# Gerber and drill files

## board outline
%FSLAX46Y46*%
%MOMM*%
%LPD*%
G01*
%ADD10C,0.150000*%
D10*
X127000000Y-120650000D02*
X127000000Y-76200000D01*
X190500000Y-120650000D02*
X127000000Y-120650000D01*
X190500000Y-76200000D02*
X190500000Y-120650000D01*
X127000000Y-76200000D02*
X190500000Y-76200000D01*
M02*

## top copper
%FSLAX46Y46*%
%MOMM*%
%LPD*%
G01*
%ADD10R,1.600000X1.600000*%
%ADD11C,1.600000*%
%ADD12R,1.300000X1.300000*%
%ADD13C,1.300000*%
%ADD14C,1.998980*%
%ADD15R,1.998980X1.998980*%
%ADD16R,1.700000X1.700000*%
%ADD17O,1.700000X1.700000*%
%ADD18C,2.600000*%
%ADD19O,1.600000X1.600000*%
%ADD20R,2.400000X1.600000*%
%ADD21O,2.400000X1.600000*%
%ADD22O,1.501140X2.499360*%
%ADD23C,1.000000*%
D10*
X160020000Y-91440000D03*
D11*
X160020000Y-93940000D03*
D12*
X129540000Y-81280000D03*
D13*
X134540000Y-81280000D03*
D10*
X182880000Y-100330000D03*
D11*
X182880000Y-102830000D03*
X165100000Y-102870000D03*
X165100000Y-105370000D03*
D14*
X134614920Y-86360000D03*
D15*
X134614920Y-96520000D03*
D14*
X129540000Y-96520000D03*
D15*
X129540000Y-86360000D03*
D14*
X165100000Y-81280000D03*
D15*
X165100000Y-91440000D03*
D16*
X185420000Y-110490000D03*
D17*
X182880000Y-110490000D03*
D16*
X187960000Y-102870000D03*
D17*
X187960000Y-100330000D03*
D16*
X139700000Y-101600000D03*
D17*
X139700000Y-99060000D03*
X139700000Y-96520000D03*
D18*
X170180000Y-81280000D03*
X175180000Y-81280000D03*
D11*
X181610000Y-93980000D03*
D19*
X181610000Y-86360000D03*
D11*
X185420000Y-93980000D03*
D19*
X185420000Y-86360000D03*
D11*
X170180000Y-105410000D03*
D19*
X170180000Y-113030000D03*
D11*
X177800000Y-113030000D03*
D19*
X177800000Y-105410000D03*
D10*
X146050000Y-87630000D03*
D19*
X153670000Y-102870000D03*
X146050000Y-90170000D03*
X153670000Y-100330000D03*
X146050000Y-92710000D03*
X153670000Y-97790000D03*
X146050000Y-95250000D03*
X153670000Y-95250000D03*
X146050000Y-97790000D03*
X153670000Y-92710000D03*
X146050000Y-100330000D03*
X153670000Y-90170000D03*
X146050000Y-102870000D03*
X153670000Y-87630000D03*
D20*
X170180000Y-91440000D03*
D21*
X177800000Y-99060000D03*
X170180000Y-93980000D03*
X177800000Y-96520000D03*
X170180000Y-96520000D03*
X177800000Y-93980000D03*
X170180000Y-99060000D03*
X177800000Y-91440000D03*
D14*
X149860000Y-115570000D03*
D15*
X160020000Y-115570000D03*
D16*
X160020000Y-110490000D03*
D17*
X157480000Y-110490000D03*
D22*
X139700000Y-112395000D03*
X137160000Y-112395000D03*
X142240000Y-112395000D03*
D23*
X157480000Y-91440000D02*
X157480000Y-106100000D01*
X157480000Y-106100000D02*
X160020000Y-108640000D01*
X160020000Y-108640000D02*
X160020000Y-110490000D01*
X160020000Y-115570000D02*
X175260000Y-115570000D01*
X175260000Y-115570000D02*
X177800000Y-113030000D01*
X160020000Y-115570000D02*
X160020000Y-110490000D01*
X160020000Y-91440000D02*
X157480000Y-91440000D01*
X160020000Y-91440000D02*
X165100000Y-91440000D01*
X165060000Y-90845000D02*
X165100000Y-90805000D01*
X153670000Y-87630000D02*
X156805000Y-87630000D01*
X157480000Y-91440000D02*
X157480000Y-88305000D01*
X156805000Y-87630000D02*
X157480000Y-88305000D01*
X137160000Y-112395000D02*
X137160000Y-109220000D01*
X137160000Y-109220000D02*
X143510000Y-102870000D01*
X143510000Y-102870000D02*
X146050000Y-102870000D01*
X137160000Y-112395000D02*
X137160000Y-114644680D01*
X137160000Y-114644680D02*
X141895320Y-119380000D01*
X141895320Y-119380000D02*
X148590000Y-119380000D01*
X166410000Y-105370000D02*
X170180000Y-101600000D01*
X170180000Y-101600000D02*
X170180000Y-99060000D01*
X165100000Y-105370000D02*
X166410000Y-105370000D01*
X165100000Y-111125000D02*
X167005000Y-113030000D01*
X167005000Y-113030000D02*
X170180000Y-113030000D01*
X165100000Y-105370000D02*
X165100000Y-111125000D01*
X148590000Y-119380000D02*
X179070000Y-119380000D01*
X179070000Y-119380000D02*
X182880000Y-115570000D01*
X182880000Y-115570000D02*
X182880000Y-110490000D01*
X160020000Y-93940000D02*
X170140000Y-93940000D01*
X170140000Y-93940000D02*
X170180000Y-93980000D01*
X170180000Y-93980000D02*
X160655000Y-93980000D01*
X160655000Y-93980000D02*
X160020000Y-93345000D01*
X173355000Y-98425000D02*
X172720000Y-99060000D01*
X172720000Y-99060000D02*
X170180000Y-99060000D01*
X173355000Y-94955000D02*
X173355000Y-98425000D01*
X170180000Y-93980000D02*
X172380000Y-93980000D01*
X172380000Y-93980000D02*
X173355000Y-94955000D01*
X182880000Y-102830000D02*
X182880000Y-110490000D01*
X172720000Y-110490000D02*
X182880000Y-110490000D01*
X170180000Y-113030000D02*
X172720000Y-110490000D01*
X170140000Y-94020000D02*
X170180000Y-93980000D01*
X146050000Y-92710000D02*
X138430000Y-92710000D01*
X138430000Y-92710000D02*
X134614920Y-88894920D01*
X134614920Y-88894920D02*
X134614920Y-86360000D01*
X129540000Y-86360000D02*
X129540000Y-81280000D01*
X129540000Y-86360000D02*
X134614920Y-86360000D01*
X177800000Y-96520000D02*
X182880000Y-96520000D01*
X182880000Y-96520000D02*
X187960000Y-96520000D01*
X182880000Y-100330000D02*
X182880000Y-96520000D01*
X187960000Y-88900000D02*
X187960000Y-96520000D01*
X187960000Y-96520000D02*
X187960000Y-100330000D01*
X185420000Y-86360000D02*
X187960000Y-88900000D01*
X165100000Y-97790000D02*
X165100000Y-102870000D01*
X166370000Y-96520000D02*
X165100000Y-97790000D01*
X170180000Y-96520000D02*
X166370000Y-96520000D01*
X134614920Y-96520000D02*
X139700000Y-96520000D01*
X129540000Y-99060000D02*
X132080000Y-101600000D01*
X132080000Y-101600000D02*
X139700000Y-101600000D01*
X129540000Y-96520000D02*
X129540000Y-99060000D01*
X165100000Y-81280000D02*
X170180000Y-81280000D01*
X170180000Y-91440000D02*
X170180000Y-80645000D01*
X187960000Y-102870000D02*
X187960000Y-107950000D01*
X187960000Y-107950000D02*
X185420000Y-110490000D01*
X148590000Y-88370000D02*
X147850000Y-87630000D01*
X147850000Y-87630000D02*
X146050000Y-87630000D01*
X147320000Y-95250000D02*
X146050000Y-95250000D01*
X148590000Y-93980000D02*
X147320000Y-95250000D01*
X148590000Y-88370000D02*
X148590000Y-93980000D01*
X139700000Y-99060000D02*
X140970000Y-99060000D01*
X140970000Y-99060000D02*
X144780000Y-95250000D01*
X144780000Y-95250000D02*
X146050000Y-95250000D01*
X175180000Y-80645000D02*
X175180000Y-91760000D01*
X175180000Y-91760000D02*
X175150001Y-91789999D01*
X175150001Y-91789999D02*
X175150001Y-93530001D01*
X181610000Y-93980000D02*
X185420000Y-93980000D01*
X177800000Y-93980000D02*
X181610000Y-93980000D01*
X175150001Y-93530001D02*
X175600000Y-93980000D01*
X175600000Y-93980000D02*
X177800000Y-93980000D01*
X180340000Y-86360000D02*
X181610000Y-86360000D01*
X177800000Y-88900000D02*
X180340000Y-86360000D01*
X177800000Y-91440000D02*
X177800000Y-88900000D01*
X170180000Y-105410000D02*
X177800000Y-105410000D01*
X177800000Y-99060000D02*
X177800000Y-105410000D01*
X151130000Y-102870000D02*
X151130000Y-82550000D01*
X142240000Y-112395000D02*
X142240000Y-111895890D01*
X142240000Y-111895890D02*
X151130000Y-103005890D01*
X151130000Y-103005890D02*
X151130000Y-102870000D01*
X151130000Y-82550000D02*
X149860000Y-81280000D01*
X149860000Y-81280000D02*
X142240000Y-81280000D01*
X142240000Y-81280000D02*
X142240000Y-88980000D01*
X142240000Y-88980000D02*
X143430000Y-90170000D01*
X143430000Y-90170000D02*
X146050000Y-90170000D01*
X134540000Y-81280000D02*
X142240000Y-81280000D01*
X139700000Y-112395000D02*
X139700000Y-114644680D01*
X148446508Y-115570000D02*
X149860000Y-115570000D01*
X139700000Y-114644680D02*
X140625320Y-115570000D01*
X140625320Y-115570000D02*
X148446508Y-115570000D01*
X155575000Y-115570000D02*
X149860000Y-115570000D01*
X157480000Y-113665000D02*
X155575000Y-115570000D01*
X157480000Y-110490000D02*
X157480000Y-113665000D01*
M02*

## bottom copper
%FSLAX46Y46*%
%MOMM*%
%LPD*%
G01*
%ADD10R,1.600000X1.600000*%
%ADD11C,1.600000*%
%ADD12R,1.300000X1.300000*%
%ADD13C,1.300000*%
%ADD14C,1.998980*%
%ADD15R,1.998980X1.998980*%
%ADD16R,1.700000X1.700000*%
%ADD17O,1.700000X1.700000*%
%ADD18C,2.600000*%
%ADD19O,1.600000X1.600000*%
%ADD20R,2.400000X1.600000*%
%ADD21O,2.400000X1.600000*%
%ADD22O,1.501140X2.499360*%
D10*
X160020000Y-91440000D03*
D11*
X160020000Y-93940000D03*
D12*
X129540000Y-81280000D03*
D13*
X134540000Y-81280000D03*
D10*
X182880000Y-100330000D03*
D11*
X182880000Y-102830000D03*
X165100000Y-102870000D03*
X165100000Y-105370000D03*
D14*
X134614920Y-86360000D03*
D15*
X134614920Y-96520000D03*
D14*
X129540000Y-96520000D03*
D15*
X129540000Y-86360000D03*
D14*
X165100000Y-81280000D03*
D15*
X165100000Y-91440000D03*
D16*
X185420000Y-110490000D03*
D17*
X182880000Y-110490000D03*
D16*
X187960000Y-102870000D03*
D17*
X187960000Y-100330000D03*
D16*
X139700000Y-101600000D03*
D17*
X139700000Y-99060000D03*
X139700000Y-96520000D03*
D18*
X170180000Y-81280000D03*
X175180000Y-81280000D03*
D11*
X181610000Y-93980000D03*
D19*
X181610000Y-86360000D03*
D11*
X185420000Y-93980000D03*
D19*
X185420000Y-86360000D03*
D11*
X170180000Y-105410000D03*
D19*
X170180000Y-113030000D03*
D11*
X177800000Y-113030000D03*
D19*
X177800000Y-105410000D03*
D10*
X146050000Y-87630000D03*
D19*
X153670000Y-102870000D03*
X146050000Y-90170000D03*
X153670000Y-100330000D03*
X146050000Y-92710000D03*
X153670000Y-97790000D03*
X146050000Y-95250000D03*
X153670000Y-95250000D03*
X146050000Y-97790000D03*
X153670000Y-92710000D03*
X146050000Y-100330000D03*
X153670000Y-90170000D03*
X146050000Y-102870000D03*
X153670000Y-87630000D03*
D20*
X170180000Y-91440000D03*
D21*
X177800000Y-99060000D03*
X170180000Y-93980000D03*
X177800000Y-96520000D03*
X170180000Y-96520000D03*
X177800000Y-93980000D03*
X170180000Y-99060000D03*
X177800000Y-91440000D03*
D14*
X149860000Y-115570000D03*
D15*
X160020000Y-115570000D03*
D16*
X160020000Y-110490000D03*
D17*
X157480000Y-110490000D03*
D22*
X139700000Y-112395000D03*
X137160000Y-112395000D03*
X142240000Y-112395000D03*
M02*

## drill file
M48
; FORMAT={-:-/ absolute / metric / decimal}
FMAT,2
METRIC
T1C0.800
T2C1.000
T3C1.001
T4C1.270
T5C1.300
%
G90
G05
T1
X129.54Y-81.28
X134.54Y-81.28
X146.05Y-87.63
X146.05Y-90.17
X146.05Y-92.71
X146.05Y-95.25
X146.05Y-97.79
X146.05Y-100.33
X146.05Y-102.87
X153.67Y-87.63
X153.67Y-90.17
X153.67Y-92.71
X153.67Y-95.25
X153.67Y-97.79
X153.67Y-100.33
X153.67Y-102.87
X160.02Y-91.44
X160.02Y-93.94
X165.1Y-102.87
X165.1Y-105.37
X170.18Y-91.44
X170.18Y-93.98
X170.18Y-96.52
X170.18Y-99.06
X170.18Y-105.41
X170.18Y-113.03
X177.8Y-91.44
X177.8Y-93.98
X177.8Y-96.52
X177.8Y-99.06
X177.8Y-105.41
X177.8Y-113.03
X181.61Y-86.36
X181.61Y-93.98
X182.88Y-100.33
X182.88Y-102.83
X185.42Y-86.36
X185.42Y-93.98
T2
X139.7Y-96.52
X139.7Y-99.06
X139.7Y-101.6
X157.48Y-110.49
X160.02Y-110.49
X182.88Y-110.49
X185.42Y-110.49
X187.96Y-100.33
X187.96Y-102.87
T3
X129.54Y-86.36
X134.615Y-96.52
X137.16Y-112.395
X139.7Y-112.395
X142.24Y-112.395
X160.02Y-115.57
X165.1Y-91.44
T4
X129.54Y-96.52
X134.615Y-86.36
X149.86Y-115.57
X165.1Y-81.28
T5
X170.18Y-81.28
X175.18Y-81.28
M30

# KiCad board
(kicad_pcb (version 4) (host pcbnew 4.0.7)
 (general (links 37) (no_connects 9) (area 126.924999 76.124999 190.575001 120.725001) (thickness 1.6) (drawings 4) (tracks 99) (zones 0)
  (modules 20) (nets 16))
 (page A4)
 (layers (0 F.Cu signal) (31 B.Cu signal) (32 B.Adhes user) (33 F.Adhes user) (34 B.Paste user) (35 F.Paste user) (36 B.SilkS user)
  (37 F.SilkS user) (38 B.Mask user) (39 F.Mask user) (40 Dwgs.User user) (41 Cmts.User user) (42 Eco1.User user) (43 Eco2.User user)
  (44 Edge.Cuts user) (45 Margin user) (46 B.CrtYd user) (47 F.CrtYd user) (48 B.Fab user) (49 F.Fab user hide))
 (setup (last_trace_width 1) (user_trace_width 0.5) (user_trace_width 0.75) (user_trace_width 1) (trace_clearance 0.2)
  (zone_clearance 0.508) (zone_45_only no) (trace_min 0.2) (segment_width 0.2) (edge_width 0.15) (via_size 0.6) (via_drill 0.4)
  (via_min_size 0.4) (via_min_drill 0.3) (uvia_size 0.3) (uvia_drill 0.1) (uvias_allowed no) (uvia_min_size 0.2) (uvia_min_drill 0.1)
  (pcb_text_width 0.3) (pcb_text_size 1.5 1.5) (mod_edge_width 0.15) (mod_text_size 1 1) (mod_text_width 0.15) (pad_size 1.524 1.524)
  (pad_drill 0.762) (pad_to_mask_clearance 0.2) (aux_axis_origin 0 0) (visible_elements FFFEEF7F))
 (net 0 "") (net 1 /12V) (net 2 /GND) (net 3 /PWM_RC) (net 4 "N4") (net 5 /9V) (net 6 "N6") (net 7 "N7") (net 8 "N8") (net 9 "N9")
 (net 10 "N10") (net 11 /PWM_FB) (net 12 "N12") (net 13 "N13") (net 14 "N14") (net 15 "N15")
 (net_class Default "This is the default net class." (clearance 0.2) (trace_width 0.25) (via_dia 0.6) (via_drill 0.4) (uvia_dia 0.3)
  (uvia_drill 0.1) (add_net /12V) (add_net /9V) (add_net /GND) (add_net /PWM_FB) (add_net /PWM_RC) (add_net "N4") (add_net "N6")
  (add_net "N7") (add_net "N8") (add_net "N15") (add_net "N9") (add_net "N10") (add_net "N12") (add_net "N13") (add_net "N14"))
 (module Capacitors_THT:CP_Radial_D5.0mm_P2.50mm (layer F.Cu) (at 160.02 91.44 270)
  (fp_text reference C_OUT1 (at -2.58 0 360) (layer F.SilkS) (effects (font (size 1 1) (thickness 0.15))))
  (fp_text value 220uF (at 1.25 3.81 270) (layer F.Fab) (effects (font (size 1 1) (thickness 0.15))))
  (pad 1 thru_hole rect (at 0 0 270) (size 1.6 1.6) (drill 0.8) (layers *.Cu *.Mask) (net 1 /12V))
  (pad 2 thru_hole circle (at 2.5 0 270) (size 1.6 1.6) (drill 0.8) (layers *.Cu *.Mask) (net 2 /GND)))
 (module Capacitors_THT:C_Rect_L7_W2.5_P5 (layer F.Cu) (at 129.54 81.28)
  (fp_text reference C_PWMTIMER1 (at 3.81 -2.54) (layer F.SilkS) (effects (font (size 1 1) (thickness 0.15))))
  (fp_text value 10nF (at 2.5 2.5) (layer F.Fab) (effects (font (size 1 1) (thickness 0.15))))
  (pad 1 thru_hole rect (at 0 0) (size 1.3 1.3) (drill 0.8) (layers *.Cu *.Mask) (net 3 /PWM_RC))
  (pad 2 thru_hole circle (at 5 0) (size 1.3 1.3) (drill 0.8) (layers *.Cu *.Mask) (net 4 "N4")))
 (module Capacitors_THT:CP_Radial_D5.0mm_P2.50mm (layer F.Cu) (at 182.88 100.33 270)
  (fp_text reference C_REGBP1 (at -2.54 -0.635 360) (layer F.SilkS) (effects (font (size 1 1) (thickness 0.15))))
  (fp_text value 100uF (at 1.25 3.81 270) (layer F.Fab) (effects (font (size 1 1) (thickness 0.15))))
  (pad 1 thru_hole rect (at 0 0 270) (size 1.6 1.6) (drill 0.8) (layers *.Cu *.Mask) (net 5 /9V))
  (pad 2 thru_hole circle (at 2.5 0 270) (size 1.6 1.6) (drill 0.8) (layers *.Cu *.Mask) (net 2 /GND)))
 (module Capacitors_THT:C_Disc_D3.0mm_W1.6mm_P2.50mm (layer F.Cu) (at 165.1 102.87 270)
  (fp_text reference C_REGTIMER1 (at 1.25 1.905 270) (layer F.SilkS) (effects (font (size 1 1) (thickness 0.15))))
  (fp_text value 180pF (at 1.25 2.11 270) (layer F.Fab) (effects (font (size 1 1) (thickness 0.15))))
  (pad 1 thru_hole circle (at 0 0 270) (size 1.6 1.6) (drill 0.8) (layers *.Cu *.Mask) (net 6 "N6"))
  (pad 2 thru_hole circle (at 2.5 0 270) (size 1.6 1.6) (drill 0.8) (layers *.Cu *.Mask) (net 2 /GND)))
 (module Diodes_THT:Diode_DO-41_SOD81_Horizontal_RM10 (layer F.Cu) (at 134.61746 96.52 90)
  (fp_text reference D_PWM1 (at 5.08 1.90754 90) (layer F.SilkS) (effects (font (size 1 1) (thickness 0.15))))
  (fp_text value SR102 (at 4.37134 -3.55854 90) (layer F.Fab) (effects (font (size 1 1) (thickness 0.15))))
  (pad 2 thru_hole circle (at 10.16 -0.00254 270) (size 1.99898 1.99898) (drill 1.27) (layers *.Cu *.Mask) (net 3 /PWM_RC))
  (pad 1 thru_hole rect (at 0 -0.00254 270) (size 1.99898 1.99898) (drill 1.00076) (layers *.Cu *.Mask) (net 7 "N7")))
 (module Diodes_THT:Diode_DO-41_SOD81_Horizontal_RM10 (layer F.Cu) (at 129.53746 86.36 270)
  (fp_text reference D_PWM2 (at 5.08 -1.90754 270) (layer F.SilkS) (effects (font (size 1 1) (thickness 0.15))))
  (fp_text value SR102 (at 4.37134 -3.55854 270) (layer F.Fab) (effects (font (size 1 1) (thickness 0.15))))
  (pad 2 thru_hole circle (at 10.16 -0.00254 90) (size 1.99898 1.99898) (drill 1.27) (layers *.Cu *.Mask) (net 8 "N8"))
  (pad 1 thru_hole rect (at 0 -0.00254 90) (size 1.99898 1.99898) (drill 1.00076) (layers *.Cu *.Mask) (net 3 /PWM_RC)))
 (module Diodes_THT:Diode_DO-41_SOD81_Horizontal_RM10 (layer F.Cu) (at 165.10254 91.44 90)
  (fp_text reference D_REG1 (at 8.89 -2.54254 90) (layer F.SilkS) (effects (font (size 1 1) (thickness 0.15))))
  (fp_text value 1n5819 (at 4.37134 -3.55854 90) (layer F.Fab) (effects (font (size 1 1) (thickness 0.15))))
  (pad 2 thru_hole circle (at 10.16 -0.00254 270) (size 1.99898 1.99898) (drill 1.27) (layers *.Cu *.Mask) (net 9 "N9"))
  (pad 1 thru_hole rect (at 0 -0.00254 270) (size 1.99898 1.99898) (drill 1.00076) (layers *.Cu *.Mask) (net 1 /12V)))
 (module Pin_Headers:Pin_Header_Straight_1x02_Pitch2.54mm (layer F.Cu) (at 185.42 110.49 270)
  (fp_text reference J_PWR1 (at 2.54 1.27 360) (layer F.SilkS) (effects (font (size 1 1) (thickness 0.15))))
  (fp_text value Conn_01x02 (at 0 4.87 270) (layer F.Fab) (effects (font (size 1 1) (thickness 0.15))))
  (pad 1 thru_hole rect (at 0 0 270) (size 1.7 1.7) (drill 1) (layers *.Cu *.Mask) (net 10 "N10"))
  (pad 2 thru_hole oval (at 0 2.54 270) (size 1.7 1.7) (drill 1) (layers *.Cu *.Mask) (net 2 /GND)))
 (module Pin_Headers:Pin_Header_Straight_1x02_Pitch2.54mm (layer F.Cu) (at 187.96 102.87 180)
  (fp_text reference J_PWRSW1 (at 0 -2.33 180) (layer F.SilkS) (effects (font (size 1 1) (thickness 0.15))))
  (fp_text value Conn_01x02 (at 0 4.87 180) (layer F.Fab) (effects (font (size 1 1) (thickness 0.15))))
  (pad 1 thru_hole rect (at 0 0 180) (size 1.7 1.7) (drill 1) (layers *.Cu *.Mask) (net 10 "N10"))
  (pad 2 thru_hole oval (at 0 2.54 180) (size 1.7 1.7) (drill 1) (layers *.Cu *.Mask) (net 5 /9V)))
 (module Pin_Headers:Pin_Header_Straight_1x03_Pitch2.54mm (layer F.Cu) (at 139.7 101.6 180)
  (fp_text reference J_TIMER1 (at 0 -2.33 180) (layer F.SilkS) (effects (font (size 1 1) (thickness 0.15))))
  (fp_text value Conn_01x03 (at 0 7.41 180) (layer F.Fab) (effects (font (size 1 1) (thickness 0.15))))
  (pad 1 thru_hole rect (at 0 0 180) (size 1.7 1.7) (drill 1) (layers *.Cu *.Mask) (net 8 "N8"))
  (pad 2 thru_hole oval (at 0 2.54 180) (size 1.7 1.7) (drill 1) (layers *.Cu *.Mask) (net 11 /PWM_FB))
  (pad 3 thru_hole oval (at 0 5.08 180) (size 1.7 1.7) (drill 1) (layers *.Cu *.Mask) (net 7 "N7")))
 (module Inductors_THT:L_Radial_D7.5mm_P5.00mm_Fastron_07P (layer F.Cu) (at 170.18 81.28)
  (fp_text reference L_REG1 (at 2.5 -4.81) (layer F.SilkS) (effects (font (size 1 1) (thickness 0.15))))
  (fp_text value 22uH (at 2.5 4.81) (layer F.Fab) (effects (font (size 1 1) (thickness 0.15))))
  (pad 1 thru_hole circle (at 0 0) (size 2.6 2.6) (drill 1.3) (layers *.Cu *.Mask) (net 9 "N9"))
  (pad 2 thru_hole circle (at 5 0) (size 2.6 2.6) (drill 1.3) (layers *.Cu *.Mask) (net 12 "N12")))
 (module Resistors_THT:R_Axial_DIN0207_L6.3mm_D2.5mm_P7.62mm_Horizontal (layer F.Cu) (at 181.61 93.98 90)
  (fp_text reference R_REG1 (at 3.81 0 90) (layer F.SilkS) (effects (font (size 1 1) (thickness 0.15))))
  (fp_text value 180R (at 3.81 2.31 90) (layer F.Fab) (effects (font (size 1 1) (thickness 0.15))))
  (pad 1 thru_hole circle (at 0 0 90) (size 1.6 1.6) (drill 0.8) (layers *.Cu *.Mask) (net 12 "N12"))
  (pad 2 thru_hole oval (at 7.62 0 90) (size 1.6 1.6) (drill 0.8) (layers *.Cu *.Mask) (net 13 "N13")))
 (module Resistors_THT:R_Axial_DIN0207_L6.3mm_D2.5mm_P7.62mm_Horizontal (layer F.Cu) (at 185.42 93.98 90)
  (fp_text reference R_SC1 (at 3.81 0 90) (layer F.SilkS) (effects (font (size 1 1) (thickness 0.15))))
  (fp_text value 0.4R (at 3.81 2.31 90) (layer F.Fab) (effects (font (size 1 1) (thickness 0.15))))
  (pad 1 thru_hole circle (at 0 0 90) (size 1.6 1.6) (drill 0.8) (layers *.Cu *.Mask) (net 12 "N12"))
  (pad 2 thru_hole oval (at 7.62 0 90) (size 1.6 1.6) (drill 0.8) (layers *.Cu *.Mask) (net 5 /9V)))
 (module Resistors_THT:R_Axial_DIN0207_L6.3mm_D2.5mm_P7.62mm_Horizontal (layer F.Cu) (at 170.18 105.41 270)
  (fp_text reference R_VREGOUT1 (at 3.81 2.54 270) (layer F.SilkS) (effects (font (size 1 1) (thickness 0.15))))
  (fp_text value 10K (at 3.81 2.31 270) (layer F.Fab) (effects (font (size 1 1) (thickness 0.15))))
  (pad 1 thru_hole circle (at 0 0 270) (size 1.6 1.6) (drill 0.8) (layers *.Cu *.Mask) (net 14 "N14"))
  (pad 2 thru_hole oval (at 7.62 0 270) (size 1.6 1.6) (drill 0.8) (layers *.Cu *.Mask) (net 2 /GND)))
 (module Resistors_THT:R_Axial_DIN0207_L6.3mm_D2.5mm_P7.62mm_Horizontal (layer F.Cu) (at 177.8 113.03 90)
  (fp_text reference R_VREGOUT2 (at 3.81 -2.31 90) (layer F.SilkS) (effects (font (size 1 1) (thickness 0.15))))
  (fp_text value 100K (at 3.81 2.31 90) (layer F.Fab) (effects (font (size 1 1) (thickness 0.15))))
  (pad 1 thru_hole circle (at 0 0 90) (size 1.6 1.6) (drill 0.8) (layers *.Cu *.Mask) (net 1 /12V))
  (pad 2 thru_hole oval (at 7.62 0 90) (size 1.6 1.6) (drill 0.8) (layers *.Cu *.Mask) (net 14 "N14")))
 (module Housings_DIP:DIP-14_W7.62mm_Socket (layer F.Cu) (at 146.05 87.63)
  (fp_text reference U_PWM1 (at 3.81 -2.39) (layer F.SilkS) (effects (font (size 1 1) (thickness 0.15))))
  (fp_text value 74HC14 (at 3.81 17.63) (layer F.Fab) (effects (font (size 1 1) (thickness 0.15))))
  (pad 1 thru_hole rect (at 0 0) (size 1.6 1.6) (drill 0.8) (layers *.Cu *.Mask) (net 11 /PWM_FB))
  (pad 8 thru_hole oval (at 7.62 15.24) (size 1.6 1.6) (drill 0.8) (layers *.Cu *.Mask))
  (pad 2 thru_hole oval (at 0 2.54) (size 1.6 1.6) (drill 0.8) (layers *.Cu *.Mask) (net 4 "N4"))
  (pad 9 thru_hole oval (at 7.62 12.7) (size 1.6 1.6) (drill 0.8) (layers *.Cu *.Mask))
  (pad 3 thru_hole oval (at 0 5.08) (size 1.6 1.6) (drill 0.8) (layers *.Cu *.Mask) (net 3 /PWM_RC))
  (pad 10 thru_hole oval (at 7.62 10.16) (size 1.6 1.6) (drill 0.8) (layers *.Cu *.Mask))
  (pad 4 thru_hole oval (at 0 7.62) (size 1.6 1.6) (drill 0.8) (layers *.Cu *.Mask) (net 11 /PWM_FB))
  (pad 11 thru_hole oval (at 7.62 7.62) (size 1.6 1.6) (drill 0.8) (layers *.Cu *.Mask))
  (pad 5 thru_hole oval (at 0 10.16) (size 1.6 1.6) (drill 0.8) (layers *.Cu *.Mask))
  (pad 12 thru_hole oval (at 7.62 5.08) (size 1.6 1.6) (drill 0.8) (layers *.Cu *.Mask))
  (pad 6 thru_hole oval (at 0 12.7) (size 1.6 1.6) (drill 0.8) (layers *.Cu *.Mask))
  (pad 13 thru_hole oval (at 7.62 2.54) (size 1.6 1.6) (drill 0.8) (layers *.Cu *.Mask))
  (pad 7 thru_hole oval (at 0 15.24) (size 1.6 1.6) (drill 0.8) (layers *.Cu *.Mask) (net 2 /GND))
  (pad 14 thru_hole oval (at 7.62 0) (size 1.6 1.6) (drill 0.8) (layers *.Cu *.Mask) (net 1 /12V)))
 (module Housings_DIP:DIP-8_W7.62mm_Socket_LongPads (layer F.Cu) (at 170.18 91.44)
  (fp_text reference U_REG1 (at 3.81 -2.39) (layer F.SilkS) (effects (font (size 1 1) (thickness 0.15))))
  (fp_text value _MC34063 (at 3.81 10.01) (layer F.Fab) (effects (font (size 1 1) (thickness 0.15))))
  (pad 1 thru_hole rect (at 0 0) (size 2.4 1.6) (drill 0.8) (layers *.Cu *.Mask) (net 9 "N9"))
  (pad 5 thru_hole oval (at 7.62 7.62) (size 2.4 1.6) (drill 0.8) (layers *.Cu *.Mask) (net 14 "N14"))
  (pad 2 thru_hole oval (at 0 2.54) (size 2.4 1.6) (drill 0.8) (layers *.Cu *.Mask) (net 2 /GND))
  (pad 6 thru_hole oval (at 7.62 5.08) (size 2.4 1.6) (drill 0.8) (layers *.Cu *.Mask) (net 5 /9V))
  (pad 3 thru_hole oval (at 0 5.08) (size 2.4 1.6) (drill 0.8) (layers *.Cu *.Mask) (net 6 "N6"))
  (pad 7 thru_hole oval (at 7.62 2.54) (size 2.4 1.6) (drill 0.8) (layers *.Cu *.Mask) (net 12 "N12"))
  (pad 4 thru_hole oval (at 0 7.62) (size 2.4 1.6) (drill 0.8) (layers *.Cu *.Mask) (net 2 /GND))
  (pad 8 thru_hole oval (at 7.62 0) (size 2.4 1.6) (drill 0.8) (layers *.Cu *.Mask) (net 13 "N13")))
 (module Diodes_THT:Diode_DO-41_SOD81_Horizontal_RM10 (layer F.Cu) (at 160.02 115.56746 180)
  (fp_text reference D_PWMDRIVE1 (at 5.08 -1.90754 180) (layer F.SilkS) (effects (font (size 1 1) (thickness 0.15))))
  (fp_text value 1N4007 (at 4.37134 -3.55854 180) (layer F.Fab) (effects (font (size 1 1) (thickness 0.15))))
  (pad 2 thru_hole circle (at 10.16 -0.00254) (size 1.99898 1.99898) (drill 1.27) (layers *.Cu *.Mask) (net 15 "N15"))
  (pad 1 thru_hole rect (at 0 -0.00254) (size 1.99898 1.99898) (drill 1.00076) (layers *.Cu *.Mask) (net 1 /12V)))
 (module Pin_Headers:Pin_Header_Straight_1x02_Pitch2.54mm (layer F.Cu) (at 160.02 110.49 270)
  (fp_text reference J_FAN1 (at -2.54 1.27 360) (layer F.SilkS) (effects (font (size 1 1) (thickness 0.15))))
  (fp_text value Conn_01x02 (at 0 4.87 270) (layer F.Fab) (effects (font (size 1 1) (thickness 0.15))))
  (pad 1 thru_hole rect (at 0 0 270) (size 1.7 1.7) (drill 1) (layers *.Cu *.Mask) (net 1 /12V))
  (pad 2 thru_hole oval (at 0 2.54 270) (size 1.7 1.7) (drill 1) (layers *.Cu *.Mask) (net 15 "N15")))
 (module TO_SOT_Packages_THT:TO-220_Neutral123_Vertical (layer F.Cu) (at 139.7 112.395)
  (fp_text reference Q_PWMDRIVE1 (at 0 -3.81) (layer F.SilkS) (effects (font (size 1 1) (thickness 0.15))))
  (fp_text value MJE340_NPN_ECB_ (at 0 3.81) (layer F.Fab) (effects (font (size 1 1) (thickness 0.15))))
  (pad 2 thru_hole oval (at 0 0 90) (size 2.49936 1.50114) (drill 1.00076) (layers *.Cu *.Mask) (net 15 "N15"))
  (pad 1 thru_hole oval (at -2.54 0 90) (size 2.49936 1.50114) (drill 1.00076) (layers *.Cu *.Mask) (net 2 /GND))
  (pad 3 thru_hole oval (at 2.54 0 90) (size 2.49936 1.50114) (drill 1.00076) (layers *.Cu *.Mask) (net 4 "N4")))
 (gr_line (start 127 120.65) (end 127 76.2) (layer Edge.Cuts) (width 0.15))
 (gr_line (start 190.5 120.65) (end 127 120.65) (layer Edge.Cuts) (width 0.15))
 (gr_line (start 190.5 76.2) (end 190.5 120.65) (layer Edge.Cuts) (width 0.15))
 (gr_line (start 127 76.2) (end 190.5 76.2) (layer Edge.Cuts) (width 0.15))
 (segment (start 157.48 91.44) (end 157.48 106.1) (width 1) (layer F.Cu) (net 1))
 (segment (start 157.48 106.1) (end 160.02 108.64) (width 1) (layer F.Cu) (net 1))
 (segment (start 160.02 108.64) (end 160.02 110.49) (width 1) (layer F.Cu) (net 1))
 (segment (start 160.02 115.57) (end 175.26 115.57) (width 1) (layer F.Cu) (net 1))
 (segment (start 175.26 115.57) (end 177.8 113.03) (width 1) (layer F.Cu) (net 1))
 (segment (start 160.02 115.57) (end 160.02 110.49) (width 1) (layer F.Cu) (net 1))
 (segment (start 160.02 91.44) (end 157.48 91.44) (width 1) (layer F.Cu) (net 1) (status 10))
 (segment (start 160.02 91.44) (end 165.1 91.44) (width 1) (layer F.Cu) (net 1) (status 30))
 (segment (start 165.06 90.845) (end 165.1 90.805) (width 1) (layer F.Cu) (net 1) (status 30))
 (segment (start 153.67 87.63) (end 156.805 87.63) (width 1) (layer F.Cu) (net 1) (status 10))
 (segment (start 157.48 91.44) (end 157.48 88.305) (width 1) (layer F.Cu) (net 1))
 (segment (start 156.805 87.63) (end 157.48 88.305) (width 1) (layer F.Cu) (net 1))
 (segment (start 137.16 112.395) (end 137.16 109.22) (width 1) (layer F.Cu) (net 2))
 (segment (start 137.16 109.22) (end 143.51 102.87) (width 1) (layer F.Cu) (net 2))
 (segment (start 143.51 102.87) (end 146.05 102.87) (width 1) (layer F.Cu) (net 2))
 (segment (start 137.16 112.395) (end 137.16 114.64468) (width 1) (layer F.Cu) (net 2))
 (segment (start 137.16 114.64468) (end 141.89532 119.38) (width 1) (layer F.Cu) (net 2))
 (segment (start 141.89532 119.38) (end 148.59 119.38) (width 1) (layer F.Cu) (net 2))
 (segment (start 166.41 105.37) (end 170.18 101.6) (width 1) (layer F.Cu) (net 2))
 (segment (start 170.18 101.6) (end 170.18 99.06) (width 1) (layer F.Cu) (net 2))
 (segment (start 165.1 105.37) (end 166.41 105.37) (width 1) (layer F.Cu) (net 2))
 (segment (start 165.1 111.125) (end 167.005 113.03) (width 1) (layer F.Cu) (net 2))
 (segment (start 167.005 113.03) (end 170.18 113.03) (width 1) (layer F.Cu) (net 2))
 (segment (start 165.1 105.37) (end 165.1 111.125) (width 1) (layer F.Cu) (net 2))
 (segment (start 148.59 119.38) (end 179.07 119.38) (width 1) (layer F.Cu) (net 2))
 (segment (start 179.07 119.38) (end 182.88 115.57) (width 1) (layer F.Cu) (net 2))
 (segment (start 182.88 115.57) (end 182.88 110.49) (width 1) (layer F.Cu) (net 2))
 (segment (start 160.02 93.94) (end 170.14 93.94) (width 1) (layer F.Cu) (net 2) (status 30))
 (segment (start 170.14 93.94) (end 170.18 93.98) (width 1) (layer F.Cu) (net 2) (status 30))
 (segment (start 170.18 93.98) (end 160.655 93.98) (width 1) (layer F.Cu) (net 2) (status 30))
 (segment (start 160.655 93.98) (end 160.02 93.345) (width 1) (layer F.Cu) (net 2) (status 30))
 (segment (start 173.355 98.425) (end 172.72 99.06) (width 1) (layer F.Cu) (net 2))
 (segment (start 172.72 99.06) (end 170.18 99.06) (width 1) (layer F.Cu) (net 2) (status 20))
 (segment (start 173.355 94.955) (end 173.355 98.425) (width 1) (layer F.Cu) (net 2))
 (segment (start 170.18 93.98) (end 172.38 93.98) (width 1) (layer F.Cu) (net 2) (status 10))
 (segment (start 172.38 93.98) (end 173.355 94.955) (width 1) (layer F.Cu) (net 2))
 (segment (start 182.88 102.83) (end 182.88 110.49) (width 1) (layer F.Cu) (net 2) (status 30))
 (segment (start 172.72 110.49) (end 182.88 110.49) (width 1) (layer F.Cu) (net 2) (status 20))
 (segment (start 170.18 113.03) (end 172.72 110.49) (width 1) (layer F.Cu) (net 2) (status 10))
 (segment (start 170.14 94.02) (end 170.18 93.98) (width 1) (layer F.Cu) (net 2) (status 30))
 (segment (start 146.05 92.71) (end 138.43 92.71) (width 1) (layer F.Cu) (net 3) (status 10))
 (segment (start 138.43 92.71) (end 134.61492 88.89492) (width 1) (layer F.Cu) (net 3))
 (segment (start 134.61492 88.89492) (end 134.61492 86.36) (width 1) (layer F.Cu) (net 3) (status 20))
 (segment (start 129.54 86.36) (end 129.54 81.28) (width 1) (layer F.Cu) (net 3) (status 30))
 (segment (start 129.54 86.36) (end 134.61492 86.36) (width 1) (layer F.Cu) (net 3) (status 30))
 (segment (start 177.8 96.52) (end 182.88 96.52) (width 1) (layer F.Cu) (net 5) (status 10))
 (segment (start 182.88 96.52) (end 187.96 96.52) (width 1) (layer F.Cu) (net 5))
 (segment (start 182.88 100.33) (end 182.88 96.52) (width 1) (layer F.Cu) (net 5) (status 10))
 (segment (start 187.96 88.9) (end 187.96 96.52) (width 1) (layer F.Cu) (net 5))
 (segment (start 187.96 96.52) (end 187.96 100.33) (width 1) (layer F.Cu) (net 5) (status 20))
 (segment (start 185.42 86.36) (end 187.96 88.9) (width 1) (layer F.Cu) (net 5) (status 10))
 (segment (start 165.1 97.79) (end 165.1 102.87) (width 1) (layer F.Cu) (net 6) (status 20))
 (segment (start 166.37 96.52) (end 165.1 97.79) (width 1) (layer F.Cu) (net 6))
 (segment (start 170.18 96.52) (end 166.37 96.52) (width 1) (layer F.Cu) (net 6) (status 10))
 (segment (start 134.61492 96.52) (end 139.7 96.52) (width 1) (layer F.Cu) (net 7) (status 30))
 (segment (start 129.54 99.06) (end 132.08 101.6) (width 1) (layer F.Cu) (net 8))
 (segment (start 132.08 101.6) (end 139.7 101.6) (width 1) (layer F.Cu) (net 8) (status 20))
 (segment (start 129.54 96.52) (end 129.54 99.06) (width 1) (layer F.Cu) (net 8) (status 10))
 (segment (start 165.1 81.28) (end 170.18 81.28) (width 1) (layer F.Cu) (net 9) (status 30))
 (segment (start 170.18 91.44) (end 170.18 80.645) (width 1) (layer F.Cu) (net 9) (status 30))
 (segment (start 187.96 102.87) (end 187.96 107.95) (width 1) (layer F.Cu) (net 10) (status 10))
 (segment (start 187.96 107.95) (end 185.42 110.49) (width 1) (layer F.Cu) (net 10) (status 20))
 (segment (start 148.59 88.37) (end 147.85 87.63) (width 1) (layer F.Cu) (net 11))
 (segment (start 147.85 87.63) (end 146.05 87.63) (width 1) (layer F.Cu) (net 11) (status 20))
 (segment (start 147.32 95.25) (end 146.05 95.25) (width 1) (layer F.Cu) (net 11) (status 20))
 (segment (start 148.59 93.98) (end 147.32 95.25) (width 1) (layer F.Cu) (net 11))
 (segment (start 148.59 88.37) (end 148.59 93.98) (width 1) (layer F.Cu) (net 11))
 (segment (start 139.7 99.06) (end 140.97 99.06) (width 1) (layer F.Cu) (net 11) (status 10))
 (segment (start 140.97 99.06) (end 144.78 95.25) (width 1) (layer F.Cu) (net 11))
 (segment (start 144.78 95.25) (end 146.05 95.25) (width 1) (layer F.Cu) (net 11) (status 20))
 (segment (start 175.18 80.645) (end 175.18 91.76) (width 1) (layer F.Cu) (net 12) (status 10))
 (segment (start 175.18 91.76) (end 175.150001 91.789999) (width 1) (layer F.Cu) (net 12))
 (segment (start 175.150001 91.789999) (end 175.150001 93.530001) (width 1) (layer F.Cu) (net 12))
 (segment (start 181.61 93.98) (end 185.42 93.98) (width 1) (layer F.Cu) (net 12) (status 30))
 (segment (start 177.8 93.98) (end 181.61 93.98) (width 1) (layer F.Cu) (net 12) (status 30))
 (segment (start 175.150001 93.530001) (end 175.6 93.98) (width 1) (layer F.Cu) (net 12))
 (segment (start 175.6 93.98) (end 177.8 93.98) (width 1) (layer F.Cu) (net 12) (status 20))
 (segment (start 180.34 86.36) (end 181.61 86.36) (width 1) (layer F.Cu) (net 13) (status 20))
 (segment (start 177.8 88.9) (end 180.34 86.36) (width 1) (layer F.Cu) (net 13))
 (segment (start 177.8 91.44) (end 177.8 88.9) (width 1) (layer F.Cu) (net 13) (status 10))
 (segment (start 170.18 105.41) (end 177.8 105.41) (width 1) (layer F.Cu) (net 14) (status 30))
 (segment (start 177.8 99.06) (end 177.8 105.41) (width 1) (layer F.Cu) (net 14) (status 30))
 (segment (start 151.13 102.87) (end 151.13 82.55) (width 1) (layer F.Cu) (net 4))
 (segment (start 142.24 112.395) (end 142.24 111.89589) (width 1) (layer F.Cu) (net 4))
 (segment (start 142.24 111.89589) (end 151.13 103.00589) (width 1) (layer F.Cu) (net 4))
 (segment (start 151.13 103.00589) (end 151.13 102.87) (width 1) (layer F.Cu) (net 4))
 (segment (start 151.13 82.55) (end 149.86 81.28) (width 1) (layer F.Cu) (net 4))
 (segment (start 149.86 81.28) (end 142.24 81.28) (width 1) (layer F.Cu) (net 4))
 (segment (start 142.24 81.28) (end 142.24 88.98) (width 1) (layer F.Cu) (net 4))
 (segment (start 142.24 88.98) (end 143.43 90.17) (width 1) (layer F.Cu) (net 4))
 (segment (start 143.43 90.17) (end 146.05 90.17) (width 1) (layer F.Cu) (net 4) (status 20))
 (segment (start 134.54 81.28) (end 142.24 81.28) (width 1) (layer F.Cu) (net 4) (status 10))
 (segment (start 139.7 112.395) (end 139.7 114.64468) (width 1) (layer F.Cu) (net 15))
 (segment (start 148.446508 115.57) (end 149.86 115.57) (width 1) (layer F.Cu) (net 15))
 (segment (start 139.7 114.64468) (end 140.62532 115.57) (width 1) (layer F.Cu) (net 15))
 (segment (start 140.62532 115.57) (end 148.446508 115.57) (width 1) (layer F.Cu) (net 15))
 (segment (start 155.575 115.57) (end 149.86 115.57) (width 1) (layer F.Cu) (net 15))
 (segment (start 157.48 113.665) (end 155.575 115.57) (width 1) (layer F.Cu) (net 15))
 (segment (start 157.48 110.49) (end 157.48 113.665) (width 1) (layer F.Cu) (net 15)))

